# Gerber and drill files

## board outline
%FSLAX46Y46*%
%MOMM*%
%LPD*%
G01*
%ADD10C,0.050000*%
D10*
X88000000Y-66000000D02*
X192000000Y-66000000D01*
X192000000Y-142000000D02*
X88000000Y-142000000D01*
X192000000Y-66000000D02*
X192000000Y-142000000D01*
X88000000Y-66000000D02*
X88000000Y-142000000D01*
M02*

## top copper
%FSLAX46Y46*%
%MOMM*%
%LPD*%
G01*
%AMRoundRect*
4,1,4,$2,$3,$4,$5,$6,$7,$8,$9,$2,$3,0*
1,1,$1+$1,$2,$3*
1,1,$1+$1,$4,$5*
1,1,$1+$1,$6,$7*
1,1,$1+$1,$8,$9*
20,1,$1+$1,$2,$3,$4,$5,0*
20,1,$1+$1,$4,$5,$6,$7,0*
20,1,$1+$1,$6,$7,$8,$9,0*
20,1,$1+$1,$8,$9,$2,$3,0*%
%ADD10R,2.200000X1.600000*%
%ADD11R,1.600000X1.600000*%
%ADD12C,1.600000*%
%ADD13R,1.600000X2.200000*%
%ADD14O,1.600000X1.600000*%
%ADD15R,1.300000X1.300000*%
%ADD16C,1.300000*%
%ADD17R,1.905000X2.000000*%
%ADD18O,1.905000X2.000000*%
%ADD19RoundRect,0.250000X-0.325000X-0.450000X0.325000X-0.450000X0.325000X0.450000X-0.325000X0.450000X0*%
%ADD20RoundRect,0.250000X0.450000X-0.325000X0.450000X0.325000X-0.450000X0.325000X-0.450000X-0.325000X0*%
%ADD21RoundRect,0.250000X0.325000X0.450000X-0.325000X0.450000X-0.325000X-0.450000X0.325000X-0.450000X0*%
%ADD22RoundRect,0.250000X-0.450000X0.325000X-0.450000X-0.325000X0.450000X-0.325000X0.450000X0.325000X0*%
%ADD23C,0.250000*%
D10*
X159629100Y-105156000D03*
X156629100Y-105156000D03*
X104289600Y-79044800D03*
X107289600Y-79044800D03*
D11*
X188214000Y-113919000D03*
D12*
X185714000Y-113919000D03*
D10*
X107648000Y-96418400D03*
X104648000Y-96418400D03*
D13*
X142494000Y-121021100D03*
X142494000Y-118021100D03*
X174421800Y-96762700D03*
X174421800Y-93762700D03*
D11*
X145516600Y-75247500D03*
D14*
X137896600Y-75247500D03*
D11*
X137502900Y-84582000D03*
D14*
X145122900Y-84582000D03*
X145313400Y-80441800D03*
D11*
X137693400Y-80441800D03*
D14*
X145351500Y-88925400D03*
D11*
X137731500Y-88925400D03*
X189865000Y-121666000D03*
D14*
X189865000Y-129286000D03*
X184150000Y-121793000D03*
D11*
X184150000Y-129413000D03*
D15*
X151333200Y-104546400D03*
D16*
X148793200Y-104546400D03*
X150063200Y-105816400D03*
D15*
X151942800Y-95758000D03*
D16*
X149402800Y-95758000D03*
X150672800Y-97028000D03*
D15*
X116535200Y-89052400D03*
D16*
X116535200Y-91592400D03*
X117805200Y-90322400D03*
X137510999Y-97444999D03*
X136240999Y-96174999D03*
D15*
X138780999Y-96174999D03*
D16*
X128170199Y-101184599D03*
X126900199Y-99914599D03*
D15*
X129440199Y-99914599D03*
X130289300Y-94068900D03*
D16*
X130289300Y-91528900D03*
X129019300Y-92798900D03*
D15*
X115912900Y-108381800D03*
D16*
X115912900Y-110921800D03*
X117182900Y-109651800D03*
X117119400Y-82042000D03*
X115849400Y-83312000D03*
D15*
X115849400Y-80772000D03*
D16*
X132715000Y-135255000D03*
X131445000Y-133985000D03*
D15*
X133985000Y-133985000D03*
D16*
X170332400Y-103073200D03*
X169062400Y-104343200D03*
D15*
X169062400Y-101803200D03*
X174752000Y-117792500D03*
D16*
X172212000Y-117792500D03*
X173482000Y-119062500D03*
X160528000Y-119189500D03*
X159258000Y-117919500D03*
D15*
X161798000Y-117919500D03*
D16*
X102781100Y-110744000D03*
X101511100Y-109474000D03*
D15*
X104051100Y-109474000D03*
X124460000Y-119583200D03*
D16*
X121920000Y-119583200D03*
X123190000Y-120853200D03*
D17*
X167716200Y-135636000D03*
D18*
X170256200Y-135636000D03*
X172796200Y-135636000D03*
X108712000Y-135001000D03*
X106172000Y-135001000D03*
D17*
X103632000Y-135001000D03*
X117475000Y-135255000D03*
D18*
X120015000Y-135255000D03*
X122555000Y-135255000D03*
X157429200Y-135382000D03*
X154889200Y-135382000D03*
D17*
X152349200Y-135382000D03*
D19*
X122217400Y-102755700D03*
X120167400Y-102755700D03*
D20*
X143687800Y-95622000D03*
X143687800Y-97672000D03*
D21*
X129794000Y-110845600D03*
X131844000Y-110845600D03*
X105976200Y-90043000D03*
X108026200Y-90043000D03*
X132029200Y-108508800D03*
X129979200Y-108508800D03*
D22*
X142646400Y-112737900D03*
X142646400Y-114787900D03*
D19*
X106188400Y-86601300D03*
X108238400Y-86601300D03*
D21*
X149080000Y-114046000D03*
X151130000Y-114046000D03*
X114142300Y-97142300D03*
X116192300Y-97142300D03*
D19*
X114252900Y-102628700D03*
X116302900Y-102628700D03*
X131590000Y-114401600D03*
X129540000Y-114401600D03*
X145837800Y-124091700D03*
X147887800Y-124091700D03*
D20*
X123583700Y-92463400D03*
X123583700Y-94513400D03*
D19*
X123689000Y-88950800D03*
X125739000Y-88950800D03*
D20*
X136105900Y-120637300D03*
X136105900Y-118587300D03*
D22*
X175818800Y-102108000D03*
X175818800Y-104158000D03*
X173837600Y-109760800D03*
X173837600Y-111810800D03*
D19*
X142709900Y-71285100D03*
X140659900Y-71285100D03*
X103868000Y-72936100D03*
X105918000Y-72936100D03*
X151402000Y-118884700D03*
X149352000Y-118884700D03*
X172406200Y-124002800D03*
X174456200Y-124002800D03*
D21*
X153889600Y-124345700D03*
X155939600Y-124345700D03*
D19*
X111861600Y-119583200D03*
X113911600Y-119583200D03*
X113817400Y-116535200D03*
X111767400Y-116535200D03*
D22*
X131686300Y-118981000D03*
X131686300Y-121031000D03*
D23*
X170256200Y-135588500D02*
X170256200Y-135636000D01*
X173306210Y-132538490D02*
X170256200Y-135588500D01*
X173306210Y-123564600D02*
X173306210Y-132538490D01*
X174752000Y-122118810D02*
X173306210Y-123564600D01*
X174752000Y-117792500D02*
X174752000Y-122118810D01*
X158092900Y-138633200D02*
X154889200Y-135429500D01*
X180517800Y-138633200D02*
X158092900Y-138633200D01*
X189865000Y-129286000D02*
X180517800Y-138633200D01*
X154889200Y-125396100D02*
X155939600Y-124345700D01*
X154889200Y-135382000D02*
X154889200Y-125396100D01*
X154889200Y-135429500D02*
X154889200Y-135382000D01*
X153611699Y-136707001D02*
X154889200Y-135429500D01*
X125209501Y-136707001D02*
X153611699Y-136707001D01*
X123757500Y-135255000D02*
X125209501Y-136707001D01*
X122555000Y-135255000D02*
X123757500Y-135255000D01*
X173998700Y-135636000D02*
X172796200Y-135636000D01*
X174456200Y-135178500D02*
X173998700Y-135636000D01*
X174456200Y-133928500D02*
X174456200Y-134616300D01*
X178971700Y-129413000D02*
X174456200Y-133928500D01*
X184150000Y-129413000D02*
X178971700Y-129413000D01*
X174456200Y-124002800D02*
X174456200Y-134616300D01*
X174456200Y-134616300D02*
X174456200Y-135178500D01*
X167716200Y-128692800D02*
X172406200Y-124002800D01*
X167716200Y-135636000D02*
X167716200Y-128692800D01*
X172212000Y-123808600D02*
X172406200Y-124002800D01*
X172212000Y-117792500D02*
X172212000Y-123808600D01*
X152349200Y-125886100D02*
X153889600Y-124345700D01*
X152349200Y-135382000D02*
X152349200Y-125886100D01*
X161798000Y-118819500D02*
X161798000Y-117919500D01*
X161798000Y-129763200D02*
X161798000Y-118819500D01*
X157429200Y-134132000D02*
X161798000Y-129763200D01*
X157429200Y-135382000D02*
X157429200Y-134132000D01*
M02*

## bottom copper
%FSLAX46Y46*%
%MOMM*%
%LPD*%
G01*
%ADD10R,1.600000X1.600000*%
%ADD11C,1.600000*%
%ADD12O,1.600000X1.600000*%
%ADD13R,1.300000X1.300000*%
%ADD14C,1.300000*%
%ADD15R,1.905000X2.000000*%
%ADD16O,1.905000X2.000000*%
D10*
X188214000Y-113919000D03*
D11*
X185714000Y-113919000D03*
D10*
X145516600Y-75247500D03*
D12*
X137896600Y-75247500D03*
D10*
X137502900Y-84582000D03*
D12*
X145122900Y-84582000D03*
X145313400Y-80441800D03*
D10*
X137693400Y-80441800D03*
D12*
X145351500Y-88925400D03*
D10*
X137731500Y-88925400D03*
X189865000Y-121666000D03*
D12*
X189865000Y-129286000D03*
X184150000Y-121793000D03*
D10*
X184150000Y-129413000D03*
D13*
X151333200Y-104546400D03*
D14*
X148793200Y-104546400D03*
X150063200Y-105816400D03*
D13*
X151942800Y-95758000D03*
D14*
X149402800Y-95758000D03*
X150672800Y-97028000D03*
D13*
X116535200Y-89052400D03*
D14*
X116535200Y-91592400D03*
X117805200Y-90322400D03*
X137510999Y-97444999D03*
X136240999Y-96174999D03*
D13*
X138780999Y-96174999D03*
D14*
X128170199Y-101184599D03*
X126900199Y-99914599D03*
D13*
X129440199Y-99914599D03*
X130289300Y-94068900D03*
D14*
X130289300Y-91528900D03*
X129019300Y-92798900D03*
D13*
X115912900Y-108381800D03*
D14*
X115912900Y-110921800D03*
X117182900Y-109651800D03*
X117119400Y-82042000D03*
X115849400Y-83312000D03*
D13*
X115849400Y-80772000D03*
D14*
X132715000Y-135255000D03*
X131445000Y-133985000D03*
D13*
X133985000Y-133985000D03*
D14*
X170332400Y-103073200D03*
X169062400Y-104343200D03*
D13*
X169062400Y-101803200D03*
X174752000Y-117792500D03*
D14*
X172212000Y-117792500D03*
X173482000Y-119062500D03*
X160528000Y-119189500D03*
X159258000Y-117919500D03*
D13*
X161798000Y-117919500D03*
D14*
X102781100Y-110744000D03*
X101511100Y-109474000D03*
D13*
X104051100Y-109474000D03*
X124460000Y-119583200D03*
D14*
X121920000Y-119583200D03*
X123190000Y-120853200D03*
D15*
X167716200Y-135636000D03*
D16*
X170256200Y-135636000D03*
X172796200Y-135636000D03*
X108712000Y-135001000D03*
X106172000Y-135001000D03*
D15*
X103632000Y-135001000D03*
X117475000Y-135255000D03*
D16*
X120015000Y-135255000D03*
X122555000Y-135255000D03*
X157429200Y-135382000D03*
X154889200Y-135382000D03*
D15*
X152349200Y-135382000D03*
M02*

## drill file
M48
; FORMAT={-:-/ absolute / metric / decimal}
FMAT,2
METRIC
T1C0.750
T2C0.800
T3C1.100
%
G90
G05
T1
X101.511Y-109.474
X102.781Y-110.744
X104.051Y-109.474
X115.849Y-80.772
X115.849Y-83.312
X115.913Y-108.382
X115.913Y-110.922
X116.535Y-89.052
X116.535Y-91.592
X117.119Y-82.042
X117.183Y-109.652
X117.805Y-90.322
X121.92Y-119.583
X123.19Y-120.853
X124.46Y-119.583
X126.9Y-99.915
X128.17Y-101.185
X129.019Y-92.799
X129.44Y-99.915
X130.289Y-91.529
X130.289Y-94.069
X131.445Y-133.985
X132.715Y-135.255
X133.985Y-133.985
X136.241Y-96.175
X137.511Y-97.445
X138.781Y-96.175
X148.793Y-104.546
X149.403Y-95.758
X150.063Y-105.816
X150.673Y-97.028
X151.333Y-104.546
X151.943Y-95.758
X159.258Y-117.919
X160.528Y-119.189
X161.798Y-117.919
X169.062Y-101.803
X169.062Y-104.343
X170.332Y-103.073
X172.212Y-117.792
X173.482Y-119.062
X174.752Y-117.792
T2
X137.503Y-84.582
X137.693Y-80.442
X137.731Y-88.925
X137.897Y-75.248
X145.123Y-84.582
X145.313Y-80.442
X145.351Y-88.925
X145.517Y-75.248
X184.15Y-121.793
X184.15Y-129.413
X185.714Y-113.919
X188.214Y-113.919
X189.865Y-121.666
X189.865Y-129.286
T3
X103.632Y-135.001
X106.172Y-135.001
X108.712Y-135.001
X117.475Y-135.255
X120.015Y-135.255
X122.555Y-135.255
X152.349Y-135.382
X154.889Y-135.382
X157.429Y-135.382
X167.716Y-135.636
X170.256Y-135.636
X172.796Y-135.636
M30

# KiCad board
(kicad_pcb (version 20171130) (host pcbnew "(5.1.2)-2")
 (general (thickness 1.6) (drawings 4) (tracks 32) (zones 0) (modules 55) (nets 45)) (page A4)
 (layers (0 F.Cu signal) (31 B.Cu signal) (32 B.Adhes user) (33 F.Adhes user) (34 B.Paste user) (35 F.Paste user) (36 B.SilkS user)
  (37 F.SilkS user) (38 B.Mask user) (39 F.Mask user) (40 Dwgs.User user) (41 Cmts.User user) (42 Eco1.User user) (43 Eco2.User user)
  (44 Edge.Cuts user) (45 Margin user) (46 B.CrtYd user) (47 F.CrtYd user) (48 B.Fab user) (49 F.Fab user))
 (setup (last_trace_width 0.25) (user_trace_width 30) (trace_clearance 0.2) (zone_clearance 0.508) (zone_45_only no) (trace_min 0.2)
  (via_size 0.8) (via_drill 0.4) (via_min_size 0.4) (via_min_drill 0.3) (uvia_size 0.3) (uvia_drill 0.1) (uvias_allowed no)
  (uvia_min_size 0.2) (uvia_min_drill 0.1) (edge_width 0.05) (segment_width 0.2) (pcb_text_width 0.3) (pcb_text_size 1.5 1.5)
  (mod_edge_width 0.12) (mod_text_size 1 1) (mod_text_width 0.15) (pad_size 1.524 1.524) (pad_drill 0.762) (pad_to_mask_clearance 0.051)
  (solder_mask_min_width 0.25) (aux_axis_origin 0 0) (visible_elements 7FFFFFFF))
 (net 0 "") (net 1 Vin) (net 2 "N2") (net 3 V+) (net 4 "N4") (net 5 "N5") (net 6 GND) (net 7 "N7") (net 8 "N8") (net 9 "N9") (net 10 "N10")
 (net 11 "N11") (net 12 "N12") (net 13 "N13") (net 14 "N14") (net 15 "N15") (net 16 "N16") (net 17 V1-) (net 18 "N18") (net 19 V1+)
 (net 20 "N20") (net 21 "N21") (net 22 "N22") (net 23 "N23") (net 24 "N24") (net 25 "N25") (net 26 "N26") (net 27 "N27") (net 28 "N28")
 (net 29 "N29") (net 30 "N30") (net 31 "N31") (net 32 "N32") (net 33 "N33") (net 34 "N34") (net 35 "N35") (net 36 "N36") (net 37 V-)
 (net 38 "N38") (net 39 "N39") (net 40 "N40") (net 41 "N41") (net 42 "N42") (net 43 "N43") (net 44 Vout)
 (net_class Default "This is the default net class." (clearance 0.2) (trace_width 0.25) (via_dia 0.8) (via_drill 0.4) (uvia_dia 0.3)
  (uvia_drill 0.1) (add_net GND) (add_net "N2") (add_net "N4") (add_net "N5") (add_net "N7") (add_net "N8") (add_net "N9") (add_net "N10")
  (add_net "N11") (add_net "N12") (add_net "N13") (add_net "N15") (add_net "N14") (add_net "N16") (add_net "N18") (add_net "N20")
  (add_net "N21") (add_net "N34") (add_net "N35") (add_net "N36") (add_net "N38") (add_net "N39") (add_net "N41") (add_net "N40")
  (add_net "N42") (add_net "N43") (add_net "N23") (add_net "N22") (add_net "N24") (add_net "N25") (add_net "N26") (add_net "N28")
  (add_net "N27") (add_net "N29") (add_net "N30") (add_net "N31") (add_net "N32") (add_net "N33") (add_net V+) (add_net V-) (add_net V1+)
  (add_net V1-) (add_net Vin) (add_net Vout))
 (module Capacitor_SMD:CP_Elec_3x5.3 (layer F.Cu) (at 158.1291 105.156)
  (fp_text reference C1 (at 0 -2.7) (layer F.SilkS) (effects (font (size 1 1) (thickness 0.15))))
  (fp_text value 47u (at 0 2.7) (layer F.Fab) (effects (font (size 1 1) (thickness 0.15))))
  (pad 2 smd rect (at 1.5 0) (size 2.2 1.6) (layers F.Cu F.Paste F.Mask) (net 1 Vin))
  (pad 1 smd rect (at -1.5 0) (size 2.2 1.6) (layers F.Cu F.Paste F.Mask) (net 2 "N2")))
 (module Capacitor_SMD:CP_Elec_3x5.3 (layer F.Cu) (at 105.7896 79.0448 180)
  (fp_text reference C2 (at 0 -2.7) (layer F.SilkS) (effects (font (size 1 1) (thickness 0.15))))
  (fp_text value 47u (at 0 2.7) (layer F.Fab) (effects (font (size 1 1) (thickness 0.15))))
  (pad 2 smd rect (at 1.5 0 180) (size 2.2 1.6) (layers F.Cu F.Paste F.Mask) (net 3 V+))
  (pad 1 smd rect (at -1.5 0 180) (size 2.2 1.6) (layers F.Cu F.Paste F.Mask) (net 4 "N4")))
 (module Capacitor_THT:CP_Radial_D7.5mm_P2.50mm (layer F.Cu) (at 188.214 113.919 180)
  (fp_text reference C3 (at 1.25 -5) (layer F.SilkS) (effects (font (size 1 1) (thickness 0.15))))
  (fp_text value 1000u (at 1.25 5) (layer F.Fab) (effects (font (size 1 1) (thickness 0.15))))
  (pad 1 thru_hole rect (at 0 0 180) (size 1.6 1.6) (drill 0.8) (layers *.Cu *.Mask) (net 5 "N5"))
  (pad 2 thru_hole circle (at 2.5 0 180) (size 1.6 1.6) (drill 0.8) (layers *.Cu *.Mask) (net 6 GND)))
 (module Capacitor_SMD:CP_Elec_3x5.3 (layer F.Cu) (at 106.148 96.4184 180)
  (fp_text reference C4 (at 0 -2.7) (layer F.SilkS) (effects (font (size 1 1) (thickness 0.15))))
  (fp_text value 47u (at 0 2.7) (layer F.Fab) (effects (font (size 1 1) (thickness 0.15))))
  (pad 1 smd rect (at -1.5 0 180) (size 2.2 1.6) (layers F.Cu F.Paste F.Mask) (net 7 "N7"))
  (pad 2 smd rect (at 1.5 0 180) (size 2.2 1.6) (layers F.Cu F.Paste F.Mask) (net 3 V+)))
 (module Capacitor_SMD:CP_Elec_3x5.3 (layer F.Cu) (at 142.494 119.5211 90)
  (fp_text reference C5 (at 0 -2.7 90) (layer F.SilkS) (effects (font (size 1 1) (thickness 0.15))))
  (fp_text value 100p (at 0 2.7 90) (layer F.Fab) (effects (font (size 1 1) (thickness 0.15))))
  (pad 1 smd rect (at -1.5 0 90) (size 2.2 1.6) (layers F.Cu F.Paste F.Mask) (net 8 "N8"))
  (pad 2 smd rect (at 1.5 0 90) (size 2.2 1.6) (layers F.Cu F.Paste F.Mask) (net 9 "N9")))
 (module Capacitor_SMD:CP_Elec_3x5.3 (layer F.Cu) (at 174.4218 95.2627 90)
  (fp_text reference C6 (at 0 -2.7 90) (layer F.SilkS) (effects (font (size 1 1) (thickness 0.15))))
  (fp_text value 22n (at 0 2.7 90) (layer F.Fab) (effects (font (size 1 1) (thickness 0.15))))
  (pad 1 smd rect (at -1.5 0 90) (size 2.2 1.6) (layers F.Cu F.Paste F.Mask) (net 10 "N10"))
  (pad 2 smd rect (at 1.5 0 90) (size 2.2 1.6) (layers F.Cu F.Paste F.Mask) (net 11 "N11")))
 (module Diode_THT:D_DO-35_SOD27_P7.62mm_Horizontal (layer F.Cu) (at 145.5166 75.2475 180)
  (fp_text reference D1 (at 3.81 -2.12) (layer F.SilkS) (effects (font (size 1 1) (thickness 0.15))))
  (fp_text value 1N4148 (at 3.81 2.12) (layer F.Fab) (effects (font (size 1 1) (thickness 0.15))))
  (pad 1 thru_hole rect (at 0 0 180) (size 1.6 1.6) (drill 0.8) (layers *.Cu *.Mask) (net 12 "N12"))
  (pad 2 thru_hole oval (at 7.62 0 180) (size 1.6 1.6) (drill 0.8) (layers *.Cu *.Mask) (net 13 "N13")))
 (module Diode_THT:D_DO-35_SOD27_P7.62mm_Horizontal (layer F.Cu) (at 137.5029 84.582)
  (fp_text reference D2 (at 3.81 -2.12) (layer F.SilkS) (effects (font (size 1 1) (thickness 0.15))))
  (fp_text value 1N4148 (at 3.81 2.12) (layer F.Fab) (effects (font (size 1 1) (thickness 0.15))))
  (pad 1 thru_hole rect (at 0 0) (size 1.6 1.6) (drill 0.8) (layers *.Cu *.Mask) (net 8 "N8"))
  (pad 2 thru_hole oval (at 7.62 0) (size 1.6 1.6) (drill 0.8) (layers *.Cu *.Mask) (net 10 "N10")))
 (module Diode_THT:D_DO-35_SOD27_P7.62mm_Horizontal (layer F.Cu) (at 137.6934 80.4418)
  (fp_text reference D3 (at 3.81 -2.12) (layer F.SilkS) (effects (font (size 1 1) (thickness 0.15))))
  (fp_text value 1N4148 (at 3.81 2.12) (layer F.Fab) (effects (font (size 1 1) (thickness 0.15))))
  (pad 2 thru_hole oval (at 7.62 0) (size 1.6 1.6) (drill 0.8) (layers *.Cu *.Mask) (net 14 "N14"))
  (pad 1 thru_hole rect (at 0 0) (size 1.6 1.6) (drill 0.8) (layers *.Cu *.Mask) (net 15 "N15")))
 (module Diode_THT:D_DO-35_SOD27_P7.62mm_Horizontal (layer F.Cu) (at 137.7315 88.9254)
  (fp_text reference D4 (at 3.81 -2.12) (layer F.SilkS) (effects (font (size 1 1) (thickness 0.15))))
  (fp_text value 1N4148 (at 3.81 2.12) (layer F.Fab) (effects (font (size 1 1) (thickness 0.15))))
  (pad 2 thru_hole oval (at 7.62 0) (size 1.6 1.6) (drill 0.8) (layers *.Cu *.Mask) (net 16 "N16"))
  (pad 1 thru_hole rect (at 0 0) (size 1.6 1.6) (drill 0.8) (layers *.Cu *.Mask) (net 8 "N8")))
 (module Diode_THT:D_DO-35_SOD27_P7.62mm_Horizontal (layer F.Cu) (at 189.865 121.666 270)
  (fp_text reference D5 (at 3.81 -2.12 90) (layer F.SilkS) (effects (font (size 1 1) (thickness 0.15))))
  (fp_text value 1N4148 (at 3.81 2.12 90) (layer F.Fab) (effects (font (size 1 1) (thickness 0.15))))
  (pad 1 thru_hole rect (at 0 0 270) (size 1.6 1.6) (drill 0.8) (layers *.Cu *.Mask) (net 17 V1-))
  (pad 2 thru_hole oval (at 7.62 0 270) (size 1.6 1.6) (drill 0.8) (layers *.Cu *.Mask) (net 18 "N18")))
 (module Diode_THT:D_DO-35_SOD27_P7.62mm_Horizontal (layer F.Cu) (at 184.15 129.413 90)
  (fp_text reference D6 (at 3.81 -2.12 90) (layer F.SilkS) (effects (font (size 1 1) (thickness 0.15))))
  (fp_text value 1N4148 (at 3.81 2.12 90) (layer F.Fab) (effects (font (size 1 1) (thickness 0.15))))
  (pad 2 thru_hole oval (at 7.62 0 90) (size 1.6 1.6) (drill 0.8) (layers *.Cu *.Mask) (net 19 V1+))
  (pad 1 thru_hole rect (at 0 0 90) (size 1.6 1.6) (drill 0.8) (layers *.Cu *.Mask) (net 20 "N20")))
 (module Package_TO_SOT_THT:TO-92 (layer F.Cu) (at 151.3332 104.5464 180)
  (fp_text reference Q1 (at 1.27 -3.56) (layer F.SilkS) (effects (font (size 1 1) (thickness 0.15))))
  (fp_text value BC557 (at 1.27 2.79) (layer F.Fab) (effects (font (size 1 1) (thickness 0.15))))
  (pad 1 thru_hole rect (at 0 0 270) (size 1.3 1.3) (drill 0.75) (layers *.Cu *.Mask) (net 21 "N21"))
  (pad 3 thru_hole circle (at 2.54 0 270) (size 1.3 1.3) (drill 0.75) (layers *.Cu *.Mask) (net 9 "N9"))
  (pad 2 thru_hole circle (at 1.27 -1.27 270) (size 1.3 1.3) (drill 0.75) (layers *.Cu *.Mask) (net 2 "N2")))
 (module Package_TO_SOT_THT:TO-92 (layer F.Cu) (at 151.9428 95.758 180)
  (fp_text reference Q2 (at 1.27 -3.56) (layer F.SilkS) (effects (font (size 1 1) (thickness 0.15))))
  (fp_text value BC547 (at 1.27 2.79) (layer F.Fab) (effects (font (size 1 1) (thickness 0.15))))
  (pad 1 thru_hole rect (at 0 0 270) (size 1.3 1.3) (drill 0.75) (layers *.Cu *.Mask) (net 9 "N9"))
  (pad 3 thru_hole circle (at 2.54 0 270) (size 1.3 1.3) (drill 0.75) (layers *.Cu *.Mask) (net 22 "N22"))
  (pad 2 thru_hole circle (at 1.27 -1.27 270) (size 1.3 1.3) (drill 0.75) (layers *.Cu *.Mask) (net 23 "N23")))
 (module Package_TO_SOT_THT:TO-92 (layer F.Cu) (at 116.5352 89.0524 270)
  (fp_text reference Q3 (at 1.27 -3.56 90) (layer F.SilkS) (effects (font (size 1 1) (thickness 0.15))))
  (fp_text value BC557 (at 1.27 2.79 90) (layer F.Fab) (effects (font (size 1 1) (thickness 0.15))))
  (pad 1 thru_hole rect (at 0 0) (size 1.3 1.3) (drill 0.75) (layers *.Cu *.Mask) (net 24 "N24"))
  (pad 3 thru_hole circle (at 2.54 0) (size 1.3 1.3) (drill 0.75) (layers *.Cu *.Mask) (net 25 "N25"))
  (pad 2 thru_hole circle (at 1.27 -1.27) (size 1.3 1.3) (drill 0.75) (layers *.Cu *.Mask) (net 4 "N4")))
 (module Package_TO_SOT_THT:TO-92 (layer F.Cu) (at 138.780999 96.174999 180)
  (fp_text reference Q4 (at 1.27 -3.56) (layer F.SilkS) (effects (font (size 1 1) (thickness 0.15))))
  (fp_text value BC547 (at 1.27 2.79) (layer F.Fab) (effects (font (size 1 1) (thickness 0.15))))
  (pad 2 thru_hole circle (at 1.27 -1.27 270) (size 1.3 1.3) (drill 0.75) (layers *.Cu *.Mask) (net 23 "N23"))
  (pad 3 thru_hole circle (at 2.54 0 270) (size 1.3 1.3) (drill 0.75) (layers *.Cu *.Mask) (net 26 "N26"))
  (pad 1 thru_hole rect (at 0 0 270) (size 1.3 1.3) (drill 0.75) (layers *.Cu *.Mask) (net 23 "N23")))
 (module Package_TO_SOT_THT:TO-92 (layer F.Cu) (at 129.440199 99.914599 180)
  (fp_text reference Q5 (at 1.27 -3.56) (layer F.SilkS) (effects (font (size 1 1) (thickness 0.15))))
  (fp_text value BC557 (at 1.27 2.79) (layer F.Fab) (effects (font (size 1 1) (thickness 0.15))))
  (pad 2 thru_hole circle (at 1.27 -1.27 270) (size 1.3 1.3) (drill 0.75) (layers *.Cu *.Mask) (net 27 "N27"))
  (pad 3 thru_hole circle (at 2.54 0 270) (size 1.3 1.3) (drill 0.75) (layers *.Cu *.Mask) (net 23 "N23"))
  (pad 1 thru_hole rect (at 0 0 270) (size 1.3 1.3) (drill 0.75) (layers *.Cu *.Mask) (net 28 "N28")))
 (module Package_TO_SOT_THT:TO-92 (layer F.Cu) (at 130.2893 94.0689 90)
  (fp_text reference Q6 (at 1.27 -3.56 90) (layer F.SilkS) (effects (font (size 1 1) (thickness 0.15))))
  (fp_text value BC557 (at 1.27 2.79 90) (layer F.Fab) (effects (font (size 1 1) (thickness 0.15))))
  (pad 1 thru_hole rect (at 0 0 180) (size 1.3 1.3) (drill 0.75) (layers *.Cu *.Mask) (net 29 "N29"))
  (pad 3 thru_hole circle (at 2.54 0 180) (size 1.3 1.3) (drill 0.75) (layers *.Cu *.Mask) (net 3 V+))
  (pad 2 thru_hole circle (at 1.27 -1.27 180) (size 1.3 1.3) (drill 0.75) (layers *.Cu *.Mask) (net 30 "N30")))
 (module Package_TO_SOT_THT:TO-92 (layer F.Cu) (at 115.9129 108.3818 270)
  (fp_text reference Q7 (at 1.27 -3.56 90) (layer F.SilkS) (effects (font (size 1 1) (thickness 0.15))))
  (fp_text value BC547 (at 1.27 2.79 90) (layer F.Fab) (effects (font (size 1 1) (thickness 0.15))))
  (pad 1 thru_hole rect (at 0 0) (size 1.3 1.3) (drill 0.75) (layers *.Cu *.Mask) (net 6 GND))
  (pad 3 thru_hole circle (at 2.54 0) (size 1.3 1.3) (drill 0.75) (layers *.Cu *.Mask) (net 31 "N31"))
  (pad 2 thru_hole circle (at 1.27 -1.27) (size 1.3 1.3) (drill 0.75) (layers *.Cu *.Mask) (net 9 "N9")))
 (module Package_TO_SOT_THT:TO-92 (layer F.Cu) (at 115.8494 80.772 270)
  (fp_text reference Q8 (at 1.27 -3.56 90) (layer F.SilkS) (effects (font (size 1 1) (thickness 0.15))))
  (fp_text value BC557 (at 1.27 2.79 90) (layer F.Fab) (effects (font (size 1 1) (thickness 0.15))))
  (pad 2 thru_hole circle (at 1.27 -1.27) (size 1.3 1.3) (drill 0.75) (layers *.Cu *.Mask) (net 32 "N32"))
  (pad 3 thru_hole circle (at 2.54 0) (size 1.3 1.3) (drill 0.75) (layers *.Cu *.Mask) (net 15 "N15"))
  (pad 1 thru_hole rect (at 0 0) (size 1.3 1.3) (drill 0.75) (layers *.Cu *.Mask) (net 13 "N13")))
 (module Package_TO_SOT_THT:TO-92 (layer F.Cu) (at 133.985 133.985 180)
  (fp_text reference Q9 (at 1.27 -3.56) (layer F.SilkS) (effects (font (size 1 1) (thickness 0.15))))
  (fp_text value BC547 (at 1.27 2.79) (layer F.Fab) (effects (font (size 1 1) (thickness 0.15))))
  (pad 2 thru_hole circle (at 1.27 -1.27 270) (size 1.3 1.3) (drill 0.75) (layers *.Cu *.Mask) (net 31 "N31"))
  (pad 3 thru_hole circle (at 2.54 0 270) (size 1.3 1.3) (drill 0.75) (layers *.Cu *.Mask) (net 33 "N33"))
  (pad 1 thru_hole rect (at 0 0 270) (size 1.3 1.3) (drill 0.75) (layers *.Cu *.Mask) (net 8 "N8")))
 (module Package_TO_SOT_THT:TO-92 (layer F.Cu) (at 169.0624 101.8032 270)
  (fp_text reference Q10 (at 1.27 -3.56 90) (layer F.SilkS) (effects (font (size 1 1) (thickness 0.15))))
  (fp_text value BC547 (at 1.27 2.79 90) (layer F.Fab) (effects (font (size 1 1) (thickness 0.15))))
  (pad 2 thru_hole circle (at 1.27 -1.27) (size 1.3 1.3) (drill 0.75) (layers *.Cu *.Mask) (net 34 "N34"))
  (pad 3 thru_hole circle (at 2.54 0) (size 1.3 1.3) (drill 0.75) (layers *.Cu *.Mask) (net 10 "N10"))
  (pad 1 thru_hole rect (at 0 0) (size 1.3 1.3) (drill 0.75) (layers *.Cu *.Mask) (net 11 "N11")))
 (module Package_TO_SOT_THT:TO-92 (layer F.Cu) (at 174.752 117.7925 180)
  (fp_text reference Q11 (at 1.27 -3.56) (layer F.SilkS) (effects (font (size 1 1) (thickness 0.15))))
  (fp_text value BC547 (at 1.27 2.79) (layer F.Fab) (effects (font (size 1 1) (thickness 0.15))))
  (pad 1 thru_hole rect (at 0 0 270) (size 1.3 1.3) (drill 0.75) (layers *.Cu *.Mask) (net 3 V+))
  (pad 3 thru_hole circle (at 2.54 0 270) (size 1.3 1.3) (drill 0.75) (layers *.Cu *.Mask) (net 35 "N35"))
  (pad 2 thru_hole circle (at 1.27 -1.27 270) (size 1.3 1.3) (drill 0.75) (layers *.Cu *.Mask) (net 14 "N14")))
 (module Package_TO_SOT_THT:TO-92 (layer F.Cu) (at 161.798 117.9195 180)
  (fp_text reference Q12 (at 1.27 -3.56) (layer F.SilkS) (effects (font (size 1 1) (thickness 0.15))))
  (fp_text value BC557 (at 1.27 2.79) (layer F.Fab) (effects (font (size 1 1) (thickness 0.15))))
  (pad 2 thru_hole circle (at 1.27 -1.27 270) (size 1.3 1.3) (drill 0.75) (layers *.Cu *.Mask) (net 16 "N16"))
  (pad 3 thru_hole circle (at 2.54 0 270) (size 1.3 1.3) (drill 0.75) (layers *.Cu *.Mask) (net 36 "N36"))
  (pad 1 thru_hole rect (at 0 0 270) (size 1.3 1.3) (drill 0.75) (layers *.Cu *.Mask) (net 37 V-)))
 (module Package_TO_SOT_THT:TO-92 (layer F.Cu) (at 104.0511 109.474 180)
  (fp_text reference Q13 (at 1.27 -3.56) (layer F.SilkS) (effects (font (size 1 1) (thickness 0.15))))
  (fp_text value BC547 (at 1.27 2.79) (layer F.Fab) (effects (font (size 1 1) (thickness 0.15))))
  (pad 2 thru_hole circle (at 1.27 -1.27 270) (size 1.3 1.3) (drill 0.75) (layers *.Cu *.Mask) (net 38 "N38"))
  (pad 3 thru_hole circle (at 2.54 0 270) (size 1.3 1.3) (drill 0.75) (layers *.Cu *.Mask) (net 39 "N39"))
  (pad 1 thru_hole rect (at 0 0 270) (size 1.3 1.3) (drill 0.75) (layers *.Cu *.Mask) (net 3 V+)))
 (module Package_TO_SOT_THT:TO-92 (layer F.Cu) (at 124.46 119.5832 180)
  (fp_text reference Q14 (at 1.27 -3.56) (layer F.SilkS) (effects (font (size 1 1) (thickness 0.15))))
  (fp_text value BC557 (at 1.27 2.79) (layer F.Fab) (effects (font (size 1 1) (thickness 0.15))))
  (pad 1 thru_hole rect (at 0 0 270) (size 1.3 1.3) (drill 0.75) (layers *.Cu *.Mask) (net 37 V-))
  (pad 3 thru_hole circle (at 2.54 0 270) (size 1.3 1.3) (drill 0.75) (layers *.Cu *.Mask) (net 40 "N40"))
  (pad 2 thru_hole circle (at 1.27 -1.27 270) (size 1.3 1.3) (drill 0.75) (layers *.Cu *.Mask) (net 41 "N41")))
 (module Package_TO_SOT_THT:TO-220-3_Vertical (layer F.Cu) (at 167.7162 135.636)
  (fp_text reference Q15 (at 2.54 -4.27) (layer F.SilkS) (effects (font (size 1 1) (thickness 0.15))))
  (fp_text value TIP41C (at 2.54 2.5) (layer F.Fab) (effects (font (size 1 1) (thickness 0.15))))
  (pad 1 thru_hole rect (at 0 0) (size 1.905 2) (drill 1.1) (layers *.Cu *.Mask) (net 35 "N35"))
  (pad 2 thru_hole oval (at 2.54 0) (size 1.905 2) (drill 1.1) (layers *.Cu *.Mask) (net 3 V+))
  (pad 3 thru_hole oval (at 5.08 0) (size 1.905 2) (drill 1.1) (layers *.Cu *.Mask) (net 20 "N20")))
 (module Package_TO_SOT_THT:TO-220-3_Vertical (layer F.Cu) (at 103.632 135.001)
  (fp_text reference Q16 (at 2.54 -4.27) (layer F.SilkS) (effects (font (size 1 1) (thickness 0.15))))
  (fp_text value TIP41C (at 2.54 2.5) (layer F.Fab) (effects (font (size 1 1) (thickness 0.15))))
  (pad 3 thru_hole oval (at 5.08 0) (size 1.905 2) (drill 1.1) (layers *.Cu *.Mask) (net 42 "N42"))
  (pad 2 thru_hole oval (at 2.54 0) (size 1.905 2) (drill 1.1) (layers *.Cu *.Mask) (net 20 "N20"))
  (pad 1 thru_hole rect (at 0 0) (size 1.905 2) (drill 1.1) (layers *.Cu *.Mask) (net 39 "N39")))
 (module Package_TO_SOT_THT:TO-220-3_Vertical (layer F.Cu) (at 117.475 135.255)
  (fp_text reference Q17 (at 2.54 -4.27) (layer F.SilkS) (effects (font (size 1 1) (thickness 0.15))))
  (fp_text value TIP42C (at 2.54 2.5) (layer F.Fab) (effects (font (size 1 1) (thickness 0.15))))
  (pad 1 thru_hole rect (at 0 0) (size 1.905 2) (drill 1.1) (layers *.Cu *.Mask) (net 40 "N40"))
  (pad 2 thru_hole oval (at 2.54 0) (size 1.905 2) (drill 1.1) (layers *.Cu *.Mask) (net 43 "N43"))
  (pad 3 thru_hole oval (at 5.08 0) (size 1.905 2) (drill 1.1) (layers *.Cu *.Mask) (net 18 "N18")))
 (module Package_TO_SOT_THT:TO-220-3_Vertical (layer F.Cu) (at 152.3492 135.382)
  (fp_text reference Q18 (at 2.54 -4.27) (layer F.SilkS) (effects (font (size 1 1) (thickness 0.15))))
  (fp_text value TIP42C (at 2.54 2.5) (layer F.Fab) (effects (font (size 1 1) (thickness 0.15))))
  (pad 3 thru_hole oval (at 5.08 0) (size 1.905 2) (drill 1.1) (layers *.Cu *.Mask) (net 37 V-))
  (pad 2 thru_hole oval (at 2.54 0) (size 1.905 2) (drill 1.1) (layers *.Cu *.Mask) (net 18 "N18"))
  (pad 1 thru_hole rect (at 0 0) (size 1.905 2) (drill 1.1) (layers *.Cu *.Mask) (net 36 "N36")))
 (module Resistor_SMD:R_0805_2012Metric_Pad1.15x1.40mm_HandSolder (layer F.Cu) (at 121.1924 102.7557)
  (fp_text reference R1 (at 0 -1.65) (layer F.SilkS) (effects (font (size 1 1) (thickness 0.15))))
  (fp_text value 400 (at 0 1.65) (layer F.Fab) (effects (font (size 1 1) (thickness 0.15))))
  (pad 2 smd roundrect (at 1.025 0) (size 1.15 1.4) (layers F.Cu F.Paste F.Mask) (roundrect_rratio 0.217391) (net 2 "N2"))
  (pad 1 smd roundrect (at -1.025 0) (size 1.15 1.4) (layers F.Cu F.Paste F.Mask) (roundrect_rratio 0.217391) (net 6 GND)))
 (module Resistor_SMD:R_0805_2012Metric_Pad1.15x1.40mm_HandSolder (layer F.Cu) (at 143.6878 96.647 90)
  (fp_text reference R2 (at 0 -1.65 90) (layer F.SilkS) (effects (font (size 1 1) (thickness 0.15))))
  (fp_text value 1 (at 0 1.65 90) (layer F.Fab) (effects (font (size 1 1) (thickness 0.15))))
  (pad 2 smd roundrect (at 1.025 0 90) (size 1.15 1.4) (layers F.Cu F.Paste F.Mask) (roundrect_rratio 0.217391) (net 22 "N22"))
  (pad 1 smd roundrect (at -1.025 0 90) (size 1.15 1.4) (layers F.Cu F.Paste F.Mask) (roundrect_rratio 0.217391) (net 37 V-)))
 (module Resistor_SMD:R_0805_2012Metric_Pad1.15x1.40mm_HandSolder (layer F.Cu) (at 130.819 110.8456 180)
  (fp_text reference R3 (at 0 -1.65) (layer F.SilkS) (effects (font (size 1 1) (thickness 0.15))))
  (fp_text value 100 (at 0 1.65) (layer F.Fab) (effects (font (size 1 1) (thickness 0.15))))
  (pad 2 smd roundrect (at 1.025 0 180) (size 1.15 1.4) (layers F.Cu F.Paste F.Mask) (roundrect_rratio 0.217391) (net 21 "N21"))
  (pad 1 smd roundrect (at -1.025 0 180) (size 1.15 1.4) (layers F.Cu F.Paste F.Mask) (roundrect_rratio 0.217391) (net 24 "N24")))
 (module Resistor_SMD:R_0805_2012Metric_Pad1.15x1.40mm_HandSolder (layer F.Cu) (at 107.0012 90.043 180)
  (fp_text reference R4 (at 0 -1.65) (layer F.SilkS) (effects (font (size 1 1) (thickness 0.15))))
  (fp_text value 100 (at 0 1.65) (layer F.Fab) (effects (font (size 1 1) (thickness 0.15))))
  (pad 2 smd roundrect (at 1.025 0 180) (size 1.15 1.4) (layers F.Cu F.Paste F.Mask) (roundrect_rratio 0.217391) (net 3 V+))
  (pad 1 smd roundrect (at -1.025 0 180) (size 1.15 1.4) (layers F.Cu F.Paste F.Mask) (roundrect_rratio 0.217391) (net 25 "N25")))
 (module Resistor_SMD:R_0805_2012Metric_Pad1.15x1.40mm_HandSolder (layer F.Cu) (at 131.0042 108.5088 180)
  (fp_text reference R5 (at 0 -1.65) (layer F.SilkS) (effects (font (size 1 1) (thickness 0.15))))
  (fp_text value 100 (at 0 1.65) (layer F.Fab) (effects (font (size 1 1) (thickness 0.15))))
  (pad 1 smd roundrect (at -1.025 0 180) (size 1.15 1.4) (layers F.Cu F.Paste F.Mask) (roundrect_rratio 0.217391) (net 28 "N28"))
  (pad 2 smd roundrect (at 1.025 0 180) (size 1.15 1.4) (layers F.Cu F.Paste F.Mask) (roundrect_rratio 0.217391) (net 24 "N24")))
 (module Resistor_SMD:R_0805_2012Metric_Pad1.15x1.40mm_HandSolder (layer F.Cu) (at 142.6464 113.7629 270)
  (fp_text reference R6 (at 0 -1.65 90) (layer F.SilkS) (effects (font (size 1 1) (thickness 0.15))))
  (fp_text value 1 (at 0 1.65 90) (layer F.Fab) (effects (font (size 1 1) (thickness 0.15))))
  (pad 1 smd roundrect (at -1.025 0 270) (size 1.15 1.4) (layers F.Cu F.Paste F.Mask) (roundrect_rratio 0.217391) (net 26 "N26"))
  (pad 2 smd roundrect (at 1.025 0 270) (size 1.15 1.4) (layers F.Cu F.Paste F.Mask) (roundrect_rratio 0.217391) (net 37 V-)))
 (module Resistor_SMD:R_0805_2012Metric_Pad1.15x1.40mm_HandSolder (layer F.Cu) (at 107.2134 86.6013)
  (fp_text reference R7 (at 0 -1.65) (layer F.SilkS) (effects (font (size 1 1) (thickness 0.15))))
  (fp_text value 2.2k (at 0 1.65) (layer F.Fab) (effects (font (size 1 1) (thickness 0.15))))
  (pad 1 smd roundrect (at -1.025 0) (size 1.15 1.4) (layers F.Cu F.Paste F.Mask) (roundrect_rratio 0.217391) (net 4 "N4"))
  (pad 2 smd roundrect (at 1.025 0) (size 1.15 1.4) (layers F.Cu F.Paste F.Mask) (roundrect_rratio 0.217391) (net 32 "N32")))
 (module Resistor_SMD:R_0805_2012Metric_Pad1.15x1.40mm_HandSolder (layer F.Cu) (at 150.105 114.046 180)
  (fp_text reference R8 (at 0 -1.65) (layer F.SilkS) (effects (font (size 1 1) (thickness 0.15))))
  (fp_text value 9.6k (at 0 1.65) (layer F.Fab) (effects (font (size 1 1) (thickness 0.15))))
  (pad 2 smd roundrect (at 1.025 0 180) (size 1.15 1.4) (layers F.Cu F.Paste F.Mask) (roundrect_rratio 0.217391) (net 27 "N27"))
  (pad 1 smd roundrect (at -1.025 0 180) (size 1.15 1.4) (layers F.Cu F.Paste F.Mask) (roundrect_rratio 0.217391) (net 5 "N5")))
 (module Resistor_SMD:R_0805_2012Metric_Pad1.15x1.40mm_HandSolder (layer F.Cu) (at 115.1673 97.1423 180)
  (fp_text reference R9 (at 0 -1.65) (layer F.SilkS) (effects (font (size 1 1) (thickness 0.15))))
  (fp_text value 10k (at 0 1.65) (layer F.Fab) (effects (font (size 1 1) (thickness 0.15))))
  (pad 2 smd roundrect (at 1.025 0 180) (size 1.15 1.4) (layers F.Cu F.Paste F.Mask) (roundrect_rratio 0.217391) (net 7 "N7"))
  (pad 1 smd roundrect (at -1.025 0 180) (size 1.15 1.4) (layers F.Cu F.Paste F.Mask) (roundrect_rratio 0.217391) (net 29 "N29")))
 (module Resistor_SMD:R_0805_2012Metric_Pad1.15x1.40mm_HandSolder (layer F.Cu) (at 115.2779 102.6287)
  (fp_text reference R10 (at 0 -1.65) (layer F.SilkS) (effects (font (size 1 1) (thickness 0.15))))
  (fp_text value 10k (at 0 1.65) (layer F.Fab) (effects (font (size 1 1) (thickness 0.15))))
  (pad 1 smd roundrect (at -1.025 0) (size 1.15 1.4) (layers F.Cu F.Paste F.Mask) (roundrect_rratio 0.217391) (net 7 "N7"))
  (pad 2 smd roundrect (at 1.025 0) (size 1.15 1.4) (layers F.Cu F.Paste F.Mask) (roundrect_rratio 0.217391) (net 6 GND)))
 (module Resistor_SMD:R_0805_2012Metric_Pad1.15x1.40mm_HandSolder (layer F.Cu) (at 130.565 114.4016)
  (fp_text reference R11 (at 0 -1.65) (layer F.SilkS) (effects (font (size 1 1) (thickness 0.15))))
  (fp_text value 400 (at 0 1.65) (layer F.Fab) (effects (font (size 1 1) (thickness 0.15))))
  (pad 2 smd roundrect (at 1.025 0) (size 1.15 1.4) (layers F.Cu F.Paste F.Mask) (roundrect_rratio 0.217391) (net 27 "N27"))
  (pad 1 smd roundrect (at -1.025 0) (size 1.15 1.4) (layers F.Cu F.Paste F.Mask) (roundrect_rratio 0.217391) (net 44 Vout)))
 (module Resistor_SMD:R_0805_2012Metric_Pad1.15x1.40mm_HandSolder (layer F.Cu) (at 146.8628 124.0917)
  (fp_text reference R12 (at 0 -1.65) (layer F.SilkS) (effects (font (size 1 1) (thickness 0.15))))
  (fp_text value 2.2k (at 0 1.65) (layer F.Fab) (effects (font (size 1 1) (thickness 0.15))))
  (pad 1 smd roundrect (at -1.025 0) (size 1.15 1.4) (layers F.Cu F.Paste F.Mask) (roundrect_rratio 0.217391) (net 31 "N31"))
  (pad 2 smd roundrect (at 1.025 0) (size 1.15 1.4) (layers F.Cu F.Paste F.Mask) (roundrect_rratio 0.217391) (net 37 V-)))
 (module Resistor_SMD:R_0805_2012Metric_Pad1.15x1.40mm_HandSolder (layer F.Cu) (at 123.5837 93.4884 90)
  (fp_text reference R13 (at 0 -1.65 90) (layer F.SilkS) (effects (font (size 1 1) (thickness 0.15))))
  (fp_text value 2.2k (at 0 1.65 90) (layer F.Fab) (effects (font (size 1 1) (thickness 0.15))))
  (pad 2 smd roundrect (at 1.025 0 90) (size 1.15 1.4) (layers F.Cu F.Paste F.Mask) (roundrect_rratio 0.217391) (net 30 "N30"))
  (pad 1 smd roundrect (at -1.025 0 90) (size 1.15 1.4) (layers F.Cu F.Paste F.Mask) (roundrect_rratio 0.217391) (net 15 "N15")))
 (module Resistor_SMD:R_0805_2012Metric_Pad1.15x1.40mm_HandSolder (layer F.Cu) (at 124.714 88.9508)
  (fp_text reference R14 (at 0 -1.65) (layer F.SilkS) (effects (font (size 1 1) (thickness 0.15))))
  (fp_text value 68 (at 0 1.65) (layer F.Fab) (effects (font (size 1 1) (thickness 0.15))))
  (pad 1 smd roundrect (at -1.025 0) (size 1.15 1.4) (layers F.Cu F.Paste F.Mask) (roundrect_rratio 0.217391) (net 15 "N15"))
  (pad 2 smd roundrect (at 1.025 0) (size 1.15 1.4) (layers F.Cu F.Paste F.Mask) (roundrect_rratio 0.217391) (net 3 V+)))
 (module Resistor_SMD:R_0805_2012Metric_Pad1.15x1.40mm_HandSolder (layer F.Cu) (at 136.1059 119.6123 90)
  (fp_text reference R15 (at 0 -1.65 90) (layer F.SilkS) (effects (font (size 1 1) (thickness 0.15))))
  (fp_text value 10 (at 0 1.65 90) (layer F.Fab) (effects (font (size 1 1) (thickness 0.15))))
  (pad 1 smd roundrect (at -1.025 0 90) (size 1.15 1.4) (layers F.Cu F.Paste F.Mask) (roundrect_rratio 0.217391) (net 33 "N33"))
  (pad 2 smd roundrect (at 1.025 0 90) (size 1.15 1.4) (layers F.Cu F.Paste F.Mask) (roundrect_rratio 0.217391) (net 37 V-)))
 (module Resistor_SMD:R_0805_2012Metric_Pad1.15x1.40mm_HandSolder (layer F.Cu) (at 175.8188 103.133 270)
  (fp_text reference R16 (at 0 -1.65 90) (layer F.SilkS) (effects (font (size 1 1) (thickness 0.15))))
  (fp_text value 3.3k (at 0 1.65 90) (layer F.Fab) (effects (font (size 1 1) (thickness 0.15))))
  (pad 1 smd roundrect (at -1.025 0 270) (size 1.15 1.4) (layers F.Cu F.Paste F.Mask) (roundrect_rratio 0.217391) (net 12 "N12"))
  (pad 2 smd roundrect (at 1.025 0 270) (size 1.15 1.4) (layers F.Cu F.Paste F.Mask) (roundrect_rratio 0.217391) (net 34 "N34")))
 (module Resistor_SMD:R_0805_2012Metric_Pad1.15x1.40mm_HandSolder (layer F.Cu) (at 173.8376 110.7858 270)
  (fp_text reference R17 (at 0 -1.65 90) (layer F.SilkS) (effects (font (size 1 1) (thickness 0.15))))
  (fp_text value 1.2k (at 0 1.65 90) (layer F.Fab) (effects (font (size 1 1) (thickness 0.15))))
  (pad 1 smd roundrect (at -1.025 0 270) (size 1.15 1.4) (layers F.Cu F.Paste F.Mask) (roundrect_rratio 0.217391) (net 34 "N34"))
  (pad 2 smd roundrect (at 1.025 0 270) (size 1.15 1.4) (layers F.Cu F.Paste F.Mask) (roundrect_rratio 0.217391) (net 10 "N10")))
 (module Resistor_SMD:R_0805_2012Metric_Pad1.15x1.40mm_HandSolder (layer F.Cu) (at 141.6849 71.2851)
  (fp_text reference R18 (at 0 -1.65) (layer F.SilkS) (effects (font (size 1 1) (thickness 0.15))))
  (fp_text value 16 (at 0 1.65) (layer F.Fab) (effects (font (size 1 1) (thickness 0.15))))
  (pad 2 smd roundrect (at 1.025 0) (size 1.15 1.4) (layers F.Cu F.Paste F.Mask) (roundrect_rratio 0.217391) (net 11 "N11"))
  (pad 1 smd roundrect (at -1.025 0) (size 1.15 1.4) (layers F.Cu F.Paste F.Mask) (roundrect_rratio 0.217391) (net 12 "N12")))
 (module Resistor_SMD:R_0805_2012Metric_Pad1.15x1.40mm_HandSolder (layer F.Cu) (at 104.893 72.9361)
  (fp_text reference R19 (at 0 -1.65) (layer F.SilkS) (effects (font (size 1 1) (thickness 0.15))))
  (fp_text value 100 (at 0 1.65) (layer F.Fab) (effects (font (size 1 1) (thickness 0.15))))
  (pad 1 smd roundrect (at -1.025 0) (size 1.15 1.4) (layers F.Cu F.Paste F.Mask) (roundrect_rratio 0.217391) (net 38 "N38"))
  (pad 2 smd roundrect (at 1.025 0) (size 1.15 1.4) (layers F.Cu F.Paste F.Mask) (roundrect_rratio 0.217391) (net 11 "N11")))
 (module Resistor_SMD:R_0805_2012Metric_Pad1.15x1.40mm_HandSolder (layer F.Cu) (at 150.377 118.8847)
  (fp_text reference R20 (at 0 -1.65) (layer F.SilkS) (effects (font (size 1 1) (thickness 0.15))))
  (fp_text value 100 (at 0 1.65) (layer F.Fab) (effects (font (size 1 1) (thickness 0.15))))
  (pad 2 smd roundrect (at 1.025 0) (size 1.15 1.4) (layers F.Cu F.Paste F.Mask) (roundrect_rratio 0.217391) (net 10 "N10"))
  (pad 1 smd roundrect (at -1.025 0) (size 1.15 1.4) (layers F.Cu F.Paste F.Mask) (roundrect_rratio 0.217391) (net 41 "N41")))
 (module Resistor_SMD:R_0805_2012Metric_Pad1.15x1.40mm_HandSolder (layer F.Cu) (at 173.4312 124.0028)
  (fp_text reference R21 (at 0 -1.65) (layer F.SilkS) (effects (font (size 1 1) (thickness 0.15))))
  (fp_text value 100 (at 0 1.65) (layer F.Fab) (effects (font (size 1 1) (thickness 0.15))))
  (pad 1 smd roundrect (at -1.025 0) (size 1.15 1.4) (layers F.Cu F.Paste F.Mask) (roundrect_rratio 0.217391) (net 35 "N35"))
  (pad 2 smd roundrect (at 1.025 0) (size 1.15 1.4) (layers F.Cu F.Paste F.Mask) (roundrect_rratio 0.217391) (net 20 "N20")))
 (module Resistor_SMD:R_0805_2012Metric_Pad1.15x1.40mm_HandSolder (layer F.Cu) (at 154.9146 124.3457 180)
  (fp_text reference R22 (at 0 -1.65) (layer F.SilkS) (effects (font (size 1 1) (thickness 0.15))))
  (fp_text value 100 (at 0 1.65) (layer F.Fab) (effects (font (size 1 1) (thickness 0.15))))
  (pad 2 smd roundrect (at 1.025 0 180) (size 1.15 1.4) (layers F.Cu F.Paste F.Mask) (roundrect_rratio 0.217391) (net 36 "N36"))
  (pad 1 smd roundrect (at -1.025 0 180) (size 1.15 1.4) (layers F.Cu F.Paste F.Mask) (roundrect_rratio 0.217391) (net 18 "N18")))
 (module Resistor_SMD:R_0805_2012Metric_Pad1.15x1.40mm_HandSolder (layer F.Cu) (at 112.8866 119.5832)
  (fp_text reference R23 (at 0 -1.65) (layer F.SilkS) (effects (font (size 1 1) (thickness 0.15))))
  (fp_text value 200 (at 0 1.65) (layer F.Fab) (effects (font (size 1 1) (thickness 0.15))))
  (pad 1 smd roundrect (at -1.025 0) (size 1.15 1.4) (layers F.Cu F.Paste F.Mask) (roundrect_rratio 0.217391) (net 39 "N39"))
  (pad 2 smd roundrect (at 1.025 0) (size 1.15 1.4) (layers F.Cu F.Paste F.Mask) (roundrect_rratio 0.217391) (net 40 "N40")))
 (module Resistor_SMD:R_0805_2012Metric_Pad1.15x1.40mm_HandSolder (layer F.Cu) (at 112.7924 116.5352)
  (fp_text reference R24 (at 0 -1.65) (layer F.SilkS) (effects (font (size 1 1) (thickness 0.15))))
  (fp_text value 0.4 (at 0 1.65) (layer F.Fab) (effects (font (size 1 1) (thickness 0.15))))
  (pad 2 smd roundrect (at 1.025 0) (size 1.15 1.4) (layers F.Cu F.Paste F.Mask) (roundrect_rratio 0.217391) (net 44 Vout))
  (pad 1 smd roundrect (at -1.025 0) (size 1.15 1.4) (layers F.Cu F.Paste F.Mask) (roundrect_rratio 0.217391) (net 42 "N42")))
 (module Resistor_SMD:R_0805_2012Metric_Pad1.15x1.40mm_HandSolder (layer F.Cu) (at 131.6863 120.006 270)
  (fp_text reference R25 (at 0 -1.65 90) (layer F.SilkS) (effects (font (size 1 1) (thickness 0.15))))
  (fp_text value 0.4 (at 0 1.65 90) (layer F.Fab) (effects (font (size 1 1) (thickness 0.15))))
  (pad 1 smd roundrect (at -1.025 0 270) (size 1.15 1.4) (layers F.Cu F.Paste F.Mask) (roundrect_rratio 0.217391) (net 44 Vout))
  (pad 2 smd roundrect (at 1.025 0 270) (size 1.15 1.4) (layers F.Cu F.Paste F.Mask) (roundrect_rratio 0.217391) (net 43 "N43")))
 (gr_line (start 88 66) (end 192 66) (layer Edge.Cuts) (width 0.05))
 (gr_line (start 192 142) (end 88 142) (layer Edge.Cuts) (width 0.05))
 (gr_line (start 192 66) (end 192 142) (layer Edge.Cuts) (width 0.05))
 (gr_line (start 88 66) (end 88 142) (layer Edge.Cuts) (width 0.05))
 (segment (start 170.2562 135.5885) (end 170.2562 135.636) (width 0.25) (layer F.Cu) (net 3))
 (segment (start 173.30621 132.53849) (end 170.2562 135.5885) (width 0.25) (layer F.Cu) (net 3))
 (segment (start 173.30621 123.5646) (end 173.30621 132.53849) (width 0.25) (layer F.Cu) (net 3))
 (segment (start 174.752 122.11881) (end 173.30621 123.5646) (width 0.25) (layer F.Cu) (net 3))
 (segment (start 174.752 117.7925) (end 174.752 122.11881) (width 0.25) (layer F.Cu) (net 3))
 (segment (start 158.0929 138.6332) (end 154.8892 135.4295) (width 0.25) (layer F.Cu) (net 18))
 (segment (start 180.5178 138.6332) (end 158.0929 138.6332) (width 0.25) (layer F.Cu) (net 18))
 (segment (start 189.865 129.286) (end 180.5178 138.6332) (width 0.25) (layer F.Cu) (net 18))
 (segment (start 154.8892 125.3961) (end 155.9396 124.3457) (width 0.25) (layer F.Cu) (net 18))
 (segment (start 154.8892 135.382) (end 154.8892 125.3961) (width 0.25) (layer F.Cu) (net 18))
 (segment (start 154.8892 135.4295) (end 154.8892 135.382) (width 0.25) (layer F.Cu) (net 18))
 (segment (start 153.611699 136.707001) (end 154.8892 135.4295) (width 0.25) (layer F.Cu) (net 18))
 (segment (start 125.209501 136.707001) (end 153.611699 136.707001) (width 0.25) (layer F.Cu) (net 18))
 (segment (start 123.7575 135.255) (end 125.209501 136.707001) (width 0.25) (layer F.Cu) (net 18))
 (segment (start 122.555 135.255) (end 123.7575 135.255) (width 0.25) (layer F.Cu) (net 18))
 (segment (start 173.9987 135.636) (end 172.7962 135.636) (width 0.25) (layer F.Cu) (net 20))
 (segment (start 174.4562 135.1785) (end 173.9987 135.636) (width 0.25) (layer F.Cu) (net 20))
 (segment (start 174.4562 133.9285) (end 174.4562 134.6163) (width 0.25) (layer F.Cu) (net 20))
 (segment (start 178.9717 129.413) (end 174.4562 133.9285) (width 0.25) (layer F.Cu) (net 20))
 (segment (start 184.15 129.413) (end 178.9717 129.413) (width 0.25) (layer F.Cu) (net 20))
 (segment (start 174.4562 124.0028) (end 174.4562 134.6163) (width 0.25) (layer F.Cu) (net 20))
 (segment (start 174.4562 134.6163) (end 174.4562 135.1785) (width 0.25) (layer F.Cu) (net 20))
 (segment (start 167.7162 128.6928) (end 172.4062 124.0028) (width 0.25) (layer F.Cu) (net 35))
 (segment (start 167.7162 135.636) (end 167.7162 128.6928) (width 0.25) (layer F.Cu) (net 35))
 (segment (start 172.212 123.8086) (end 172.4062 124.0028) (width 0.25) (layer F.Cu) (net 35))
 (segment (start 172.212 117.7925) (end 172.212 123.8086) (width 0.25) (layer F.Cu) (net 35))
 (segment (start 152.3492 125.8861) (end 153.8896 124.3457) (width 0.25) (layer F.Cu) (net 36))
 (segment (start 152.3492 135.382) (end 152.3492 125.8861) (width 0.25) (layer F.Cu) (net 36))
 (segment (start 161.798 118.8195) (end 161.798 117.9195) (width 0.25) (layer F.Cu) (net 37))
 (segment (start 161.798 129.7632) (end 161.798 118.8195) (width 0.25) (layer F.Cu) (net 37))
 (segment (start 157.4292 134.132) (end 161.798 129.7632) (width 0.25) (layer F.Cu) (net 37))
 (segment (start 157.4292 135.382) (end 157.4292 134.132) (width 0.25) (layer F.Cu) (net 37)))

